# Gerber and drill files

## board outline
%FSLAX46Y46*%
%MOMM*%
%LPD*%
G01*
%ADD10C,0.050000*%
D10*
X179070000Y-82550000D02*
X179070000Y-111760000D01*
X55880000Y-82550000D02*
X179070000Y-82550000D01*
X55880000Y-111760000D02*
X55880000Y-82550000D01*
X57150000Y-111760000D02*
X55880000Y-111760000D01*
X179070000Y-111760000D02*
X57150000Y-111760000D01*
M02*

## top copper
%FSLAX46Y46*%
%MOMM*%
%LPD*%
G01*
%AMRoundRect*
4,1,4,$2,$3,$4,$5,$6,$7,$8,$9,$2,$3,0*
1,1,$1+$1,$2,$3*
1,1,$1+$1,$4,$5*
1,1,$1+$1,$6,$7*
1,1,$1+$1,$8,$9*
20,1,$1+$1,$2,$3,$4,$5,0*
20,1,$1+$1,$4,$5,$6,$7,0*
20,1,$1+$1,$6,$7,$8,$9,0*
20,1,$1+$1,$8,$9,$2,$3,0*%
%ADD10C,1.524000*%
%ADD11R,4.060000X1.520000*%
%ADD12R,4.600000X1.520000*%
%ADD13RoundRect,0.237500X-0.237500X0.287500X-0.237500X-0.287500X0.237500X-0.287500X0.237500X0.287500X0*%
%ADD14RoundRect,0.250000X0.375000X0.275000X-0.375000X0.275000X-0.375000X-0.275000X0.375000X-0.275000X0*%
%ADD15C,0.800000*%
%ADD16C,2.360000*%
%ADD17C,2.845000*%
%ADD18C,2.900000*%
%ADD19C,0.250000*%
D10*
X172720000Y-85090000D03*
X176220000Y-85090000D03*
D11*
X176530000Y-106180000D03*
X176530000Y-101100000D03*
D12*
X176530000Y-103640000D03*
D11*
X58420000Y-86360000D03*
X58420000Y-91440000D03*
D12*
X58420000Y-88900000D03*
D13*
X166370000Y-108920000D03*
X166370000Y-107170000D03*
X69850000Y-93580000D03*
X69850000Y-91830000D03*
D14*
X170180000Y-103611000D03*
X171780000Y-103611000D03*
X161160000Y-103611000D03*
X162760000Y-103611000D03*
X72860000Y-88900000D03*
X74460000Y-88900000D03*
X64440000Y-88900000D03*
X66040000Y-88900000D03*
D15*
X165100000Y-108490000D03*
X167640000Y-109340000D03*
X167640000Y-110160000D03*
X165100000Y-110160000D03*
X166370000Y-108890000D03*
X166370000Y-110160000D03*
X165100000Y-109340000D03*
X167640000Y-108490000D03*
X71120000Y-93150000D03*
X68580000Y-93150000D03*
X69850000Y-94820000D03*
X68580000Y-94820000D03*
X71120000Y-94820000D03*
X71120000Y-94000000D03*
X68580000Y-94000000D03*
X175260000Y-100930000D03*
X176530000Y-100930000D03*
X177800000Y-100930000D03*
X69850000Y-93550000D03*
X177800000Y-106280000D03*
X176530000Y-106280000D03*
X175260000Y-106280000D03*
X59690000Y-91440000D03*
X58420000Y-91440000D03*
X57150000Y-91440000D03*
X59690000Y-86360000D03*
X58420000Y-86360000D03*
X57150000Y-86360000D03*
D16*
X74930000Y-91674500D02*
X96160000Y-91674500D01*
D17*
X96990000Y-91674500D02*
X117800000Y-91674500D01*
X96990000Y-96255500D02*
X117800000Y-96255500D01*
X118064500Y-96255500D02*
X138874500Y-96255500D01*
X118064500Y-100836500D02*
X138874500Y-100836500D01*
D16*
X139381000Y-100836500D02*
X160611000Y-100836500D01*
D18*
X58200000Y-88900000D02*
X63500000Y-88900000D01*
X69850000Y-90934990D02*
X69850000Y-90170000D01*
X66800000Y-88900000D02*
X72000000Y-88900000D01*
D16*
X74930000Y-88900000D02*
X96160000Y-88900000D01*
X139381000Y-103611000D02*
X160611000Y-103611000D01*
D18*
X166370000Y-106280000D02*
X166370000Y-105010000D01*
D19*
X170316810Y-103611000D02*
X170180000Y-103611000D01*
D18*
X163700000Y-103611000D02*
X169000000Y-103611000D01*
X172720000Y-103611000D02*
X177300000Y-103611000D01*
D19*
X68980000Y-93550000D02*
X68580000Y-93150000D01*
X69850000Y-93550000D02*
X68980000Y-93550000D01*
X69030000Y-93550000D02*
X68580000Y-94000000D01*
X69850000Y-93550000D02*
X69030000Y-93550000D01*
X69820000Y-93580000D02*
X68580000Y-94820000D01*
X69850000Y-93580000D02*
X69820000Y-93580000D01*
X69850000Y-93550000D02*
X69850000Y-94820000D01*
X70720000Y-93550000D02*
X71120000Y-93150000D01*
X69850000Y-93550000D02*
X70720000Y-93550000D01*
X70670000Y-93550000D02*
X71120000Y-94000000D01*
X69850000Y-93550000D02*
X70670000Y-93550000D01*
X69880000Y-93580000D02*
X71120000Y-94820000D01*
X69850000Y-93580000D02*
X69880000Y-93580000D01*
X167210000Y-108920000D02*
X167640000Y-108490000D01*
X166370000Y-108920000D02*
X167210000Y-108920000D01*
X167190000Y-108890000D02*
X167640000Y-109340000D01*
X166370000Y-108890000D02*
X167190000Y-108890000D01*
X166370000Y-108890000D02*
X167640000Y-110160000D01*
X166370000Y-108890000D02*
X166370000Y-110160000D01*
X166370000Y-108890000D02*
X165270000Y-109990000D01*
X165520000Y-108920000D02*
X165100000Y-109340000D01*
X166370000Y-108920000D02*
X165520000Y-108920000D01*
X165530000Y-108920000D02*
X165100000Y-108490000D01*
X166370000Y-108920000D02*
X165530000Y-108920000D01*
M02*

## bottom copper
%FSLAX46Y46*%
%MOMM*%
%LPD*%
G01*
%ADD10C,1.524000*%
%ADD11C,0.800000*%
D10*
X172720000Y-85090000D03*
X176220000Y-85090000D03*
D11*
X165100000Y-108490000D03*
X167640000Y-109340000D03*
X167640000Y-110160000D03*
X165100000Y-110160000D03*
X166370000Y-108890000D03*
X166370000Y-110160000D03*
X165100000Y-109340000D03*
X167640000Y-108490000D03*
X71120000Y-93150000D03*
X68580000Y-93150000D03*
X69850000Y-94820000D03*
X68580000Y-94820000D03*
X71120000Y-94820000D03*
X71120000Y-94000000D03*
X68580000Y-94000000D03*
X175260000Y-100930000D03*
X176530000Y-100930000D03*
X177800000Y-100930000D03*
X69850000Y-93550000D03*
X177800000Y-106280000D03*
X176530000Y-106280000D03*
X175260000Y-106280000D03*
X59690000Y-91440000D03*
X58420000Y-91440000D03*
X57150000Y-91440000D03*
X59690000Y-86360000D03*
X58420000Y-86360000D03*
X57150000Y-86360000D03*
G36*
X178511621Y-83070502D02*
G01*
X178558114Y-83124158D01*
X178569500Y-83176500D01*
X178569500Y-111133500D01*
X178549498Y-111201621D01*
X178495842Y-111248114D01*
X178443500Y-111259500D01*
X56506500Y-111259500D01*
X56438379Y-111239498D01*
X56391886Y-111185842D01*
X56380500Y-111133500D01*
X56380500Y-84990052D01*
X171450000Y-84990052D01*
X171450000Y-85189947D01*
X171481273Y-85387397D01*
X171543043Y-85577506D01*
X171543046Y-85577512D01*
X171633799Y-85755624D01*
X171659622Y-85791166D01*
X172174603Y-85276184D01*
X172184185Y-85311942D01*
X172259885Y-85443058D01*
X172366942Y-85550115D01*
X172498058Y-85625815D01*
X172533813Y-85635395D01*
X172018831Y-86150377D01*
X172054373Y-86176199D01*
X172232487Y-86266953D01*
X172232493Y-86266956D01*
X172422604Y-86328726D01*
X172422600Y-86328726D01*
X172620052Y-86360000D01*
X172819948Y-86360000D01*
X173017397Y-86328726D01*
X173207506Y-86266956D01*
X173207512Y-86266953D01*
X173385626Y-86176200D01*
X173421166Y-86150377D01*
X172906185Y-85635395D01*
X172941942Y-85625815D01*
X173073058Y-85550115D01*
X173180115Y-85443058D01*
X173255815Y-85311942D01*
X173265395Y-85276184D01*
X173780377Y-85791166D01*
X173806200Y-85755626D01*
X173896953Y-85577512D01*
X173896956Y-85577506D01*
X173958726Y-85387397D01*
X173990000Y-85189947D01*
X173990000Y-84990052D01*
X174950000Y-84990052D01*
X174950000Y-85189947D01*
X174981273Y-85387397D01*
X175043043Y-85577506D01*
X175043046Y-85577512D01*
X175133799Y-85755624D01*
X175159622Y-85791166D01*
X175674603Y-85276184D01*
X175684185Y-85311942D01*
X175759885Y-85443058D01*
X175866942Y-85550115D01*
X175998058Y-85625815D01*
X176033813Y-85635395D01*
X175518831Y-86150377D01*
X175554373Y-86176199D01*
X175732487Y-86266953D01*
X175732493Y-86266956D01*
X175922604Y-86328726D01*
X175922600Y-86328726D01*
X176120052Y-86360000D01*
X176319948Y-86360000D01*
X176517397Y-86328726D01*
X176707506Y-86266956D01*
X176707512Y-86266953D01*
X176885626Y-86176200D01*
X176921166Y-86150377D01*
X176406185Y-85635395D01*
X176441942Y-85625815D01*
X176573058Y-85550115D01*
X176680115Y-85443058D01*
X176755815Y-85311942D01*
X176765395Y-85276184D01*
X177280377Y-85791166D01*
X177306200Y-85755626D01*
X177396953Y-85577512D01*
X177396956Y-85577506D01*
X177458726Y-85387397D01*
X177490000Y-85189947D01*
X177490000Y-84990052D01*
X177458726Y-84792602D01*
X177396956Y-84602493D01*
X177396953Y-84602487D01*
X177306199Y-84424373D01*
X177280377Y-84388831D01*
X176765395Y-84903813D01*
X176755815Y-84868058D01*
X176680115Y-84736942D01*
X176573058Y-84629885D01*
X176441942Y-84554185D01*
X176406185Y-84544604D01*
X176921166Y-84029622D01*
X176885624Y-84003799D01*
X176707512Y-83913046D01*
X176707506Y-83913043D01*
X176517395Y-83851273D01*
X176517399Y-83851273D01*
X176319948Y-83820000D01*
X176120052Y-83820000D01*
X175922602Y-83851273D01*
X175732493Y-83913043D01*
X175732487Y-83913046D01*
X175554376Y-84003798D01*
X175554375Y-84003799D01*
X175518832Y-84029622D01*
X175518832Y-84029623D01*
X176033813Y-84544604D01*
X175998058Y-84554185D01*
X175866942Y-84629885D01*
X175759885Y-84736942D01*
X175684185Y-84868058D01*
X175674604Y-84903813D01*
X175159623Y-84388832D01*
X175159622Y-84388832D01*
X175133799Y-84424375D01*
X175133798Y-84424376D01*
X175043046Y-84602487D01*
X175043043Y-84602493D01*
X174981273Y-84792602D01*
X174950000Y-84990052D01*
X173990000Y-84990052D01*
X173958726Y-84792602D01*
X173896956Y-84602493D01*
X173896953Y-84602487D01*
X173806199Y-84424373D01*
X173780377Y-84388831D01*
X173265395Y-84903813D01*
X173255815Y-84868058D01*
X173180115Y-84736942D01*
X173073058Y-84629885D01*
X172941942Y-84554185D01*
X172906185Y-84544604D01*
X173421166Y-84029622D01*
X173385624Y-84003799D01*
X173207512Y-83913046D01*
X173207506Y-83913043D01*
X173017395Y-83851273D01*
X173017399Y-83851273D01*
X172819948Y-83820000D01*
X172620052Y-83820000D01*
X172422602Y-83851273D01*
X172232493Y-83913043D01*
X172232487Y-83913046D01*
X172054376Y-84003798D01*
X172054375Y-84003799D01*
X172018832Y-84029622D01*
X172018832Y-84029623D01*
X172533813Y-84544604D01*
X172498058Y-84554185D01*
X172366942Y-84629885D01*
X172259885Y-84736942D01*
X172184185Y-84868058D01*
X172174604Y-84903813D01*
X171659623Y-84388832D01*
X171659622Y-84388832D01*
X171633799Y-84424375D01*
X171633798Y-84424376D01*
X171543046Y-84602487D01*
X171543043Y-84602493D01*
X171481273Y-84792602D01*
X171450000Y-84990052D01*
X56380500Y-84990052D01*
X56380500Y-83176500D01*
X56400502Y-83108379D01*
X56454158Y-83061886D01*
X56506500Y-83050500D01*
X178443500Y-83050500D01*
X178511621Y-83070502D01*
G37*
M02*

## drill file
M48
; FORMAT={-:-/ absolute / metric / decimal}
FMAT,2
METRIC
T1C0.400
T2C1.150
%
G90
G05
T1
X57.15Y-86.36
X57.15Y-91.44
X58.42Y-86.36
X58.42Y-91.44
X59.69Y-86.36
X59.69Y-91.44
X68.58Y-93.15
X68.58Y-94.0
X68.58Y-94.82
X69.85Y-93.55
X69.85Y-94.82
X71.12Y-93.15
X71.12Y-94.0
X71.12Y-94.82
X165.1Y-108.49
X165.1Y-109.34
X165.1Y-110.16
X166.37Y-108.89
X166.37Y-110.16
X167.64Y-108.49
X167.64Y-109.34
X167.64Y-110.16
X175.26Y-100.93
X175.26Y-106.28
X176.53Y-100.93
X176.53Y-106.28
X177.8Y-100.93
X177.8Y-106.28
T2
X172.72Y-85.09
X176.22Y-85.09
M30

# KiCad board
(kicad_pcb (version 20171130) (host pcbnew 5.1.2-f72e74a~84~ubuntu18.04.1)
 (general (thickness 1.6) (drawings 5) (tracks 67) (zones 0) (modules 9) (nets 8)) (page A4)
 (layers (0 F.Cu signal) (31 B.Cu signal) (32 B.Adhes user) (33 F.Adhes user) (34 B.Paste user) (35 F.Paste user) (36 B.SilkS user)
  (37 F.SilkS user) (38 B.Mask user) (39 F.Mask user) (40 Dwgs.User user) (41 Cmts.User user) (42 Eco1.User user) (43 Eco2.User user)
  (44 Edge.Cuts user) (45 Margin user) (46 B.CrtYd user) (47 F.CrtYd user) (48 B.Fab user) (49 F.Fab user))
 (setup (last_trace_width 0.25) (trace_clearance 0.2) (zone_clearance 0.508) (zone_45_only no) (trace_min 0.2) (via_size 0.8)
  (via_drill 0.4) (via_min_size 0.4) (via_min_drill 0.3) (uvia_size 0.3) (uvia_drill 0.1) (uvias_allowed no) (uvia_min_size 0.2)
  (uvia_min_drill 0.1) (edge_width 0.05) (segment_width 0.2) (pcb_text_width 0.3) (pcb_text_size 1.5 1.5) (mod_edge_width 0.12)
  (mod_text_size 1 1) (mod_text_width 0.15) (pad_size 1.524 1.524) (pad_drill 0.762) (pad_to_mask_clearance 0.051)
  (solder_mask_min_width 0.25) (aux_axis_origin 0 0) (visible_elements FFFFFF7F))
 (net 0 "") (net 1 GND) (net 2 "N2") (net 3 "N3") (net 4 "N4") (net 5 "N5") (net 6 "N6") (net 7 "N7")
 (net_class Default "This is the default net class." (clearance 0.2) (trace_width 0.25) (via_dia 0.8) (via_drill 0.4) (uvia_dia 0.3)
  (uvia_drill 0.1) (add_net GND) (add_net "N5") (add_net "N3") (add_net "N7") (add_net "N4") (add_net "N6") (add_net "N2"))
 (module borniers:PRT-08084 (layer F.Cu) (at 172.72 80.01 180)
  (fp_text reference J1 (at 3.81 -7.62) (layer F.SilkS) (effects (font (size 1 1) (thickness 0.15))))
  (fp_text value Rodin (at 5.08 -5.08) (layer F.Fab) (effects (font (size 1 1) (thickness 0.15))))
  (pad 2 thru_hole circle (at 0 -5.08 180) (size 1.524 1.524) (drill 1.15) (layers *.Cu *.Mask) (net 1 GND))
  (pad 1 thru_hole circle (at -3.5 -5.08 180) (size 1.524 1.524) (drill 1.15) (layers *.Cu *.Mask) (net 1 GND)))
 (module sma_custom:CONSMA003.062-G (layer F.Cu) (at 180.34 106.18)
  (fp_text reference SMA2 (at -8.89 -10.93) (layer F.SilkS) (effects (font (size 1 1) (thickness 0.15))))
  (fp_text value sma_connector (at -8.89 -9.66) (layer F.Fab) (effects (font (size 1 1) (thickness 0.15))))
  (pad 3 smd rect (at -3.81 0) (size 4.06 1.52) (layers F.Cu F.Paste F.Mask) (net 1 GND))
  (pad 2 smd rect (at -3.81 -5.08) (size 4.06 1.52) (layers F.Cu F.Paste F.Mask) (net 1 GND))
  (pad 1 smd rect (at -3.81 -2.54) (size 4.6 1.52) (layers F.Cu F.Paste F.Mask) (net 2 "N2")))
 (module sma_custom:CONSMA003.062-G (layer F.Cu) (at 54.61 86.36 180)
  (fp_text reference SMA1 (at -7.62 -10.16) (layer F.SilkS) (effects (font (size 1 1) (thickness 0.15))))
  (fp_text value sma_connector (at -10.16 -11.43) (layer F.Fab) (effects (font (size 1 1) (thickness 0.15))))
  (pad 3 smd rect (at -3.81 0 180) (size 4.06 1.52) (layers F.Cu F.Paste F.Mask) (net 1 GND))
  (pad 2 smd rect (at -3.81 -5.08 180) (size 4.06 1.52) (layers F.Cu F.Paste F.Mask) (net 1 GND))
  (pad 1 smd rect (at -3.81 -2.54 180) (size 4.6 1.52) (layers F.Cu F.Paste F.Mask) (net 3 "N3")))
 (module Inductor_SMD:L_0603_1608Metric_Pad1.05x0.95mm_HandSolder (layer F.Cu) (at 166.37 108.045 270)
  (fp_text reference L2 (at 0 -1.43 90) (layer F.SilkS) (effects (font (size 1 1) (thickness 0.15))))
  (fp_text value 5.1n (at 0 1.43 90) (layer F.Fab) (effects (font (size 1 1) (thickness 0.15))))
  (pad 2 smd roundrect (at 0.875 0 270) (size 1.05 0.95) (layers F.Cu F.Paste F.Mask) (roundrect_rratio 0.25) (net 1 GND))
  (pad 1 smd roundrect (at -0.875 0 270) (size 1.05 0.95) (layers F.Cu F.Paste F.Mask) (roundrect_rratio 0.25) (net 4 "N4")))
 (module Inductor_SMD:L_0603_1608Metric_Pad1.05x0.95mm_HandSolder (layer F.Cu) (at 69.85 92.705 270)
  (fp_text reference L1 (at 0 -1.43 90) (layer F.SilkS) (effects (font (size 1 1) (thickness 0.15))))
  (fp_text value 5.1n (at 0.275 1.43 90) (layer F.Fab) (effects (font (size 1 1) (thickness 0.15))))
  (pad 2 smd roundrect (at 0.875 0 270) (size 1.05 0.95) (layers F.Cu F.Paste F.Mask) (roundrect_rratio 0.25) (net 1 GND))
  (pad 1 smd roundrect (at -0.875 0 270) (size 1.05 0.95) (layers F.Cu F.Paste F.Mask) (roundrect_rratio 0.25) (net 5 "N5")))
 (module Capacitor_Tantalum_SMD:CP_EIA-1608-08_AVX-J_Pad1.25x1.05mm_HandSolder (layer F.Cu) (at 170.98 103.611 180)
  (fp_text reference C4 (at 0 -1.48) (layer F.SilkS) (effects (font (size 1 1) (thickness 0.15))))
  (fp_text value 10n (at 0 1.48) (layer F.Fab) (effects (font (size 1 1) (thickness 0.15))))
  (pad 2 smd roundrect (at 0.8 0 180) (size 1.25 1.05) (layers F.Cu F.Paste F.Mask) (roundrect_rratio 0.238095) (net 4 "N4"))
  (pad 1 smd roundrect (at -0.8 0 180) (size 1.25 1.05) (layers F.Cu F.Paste F.Mask) (roundrect_rratio 0.238095) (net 2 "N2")))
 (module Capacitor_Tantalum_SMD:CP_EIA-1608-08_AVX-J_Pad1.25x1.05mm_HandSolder (layer F.Cu) (at 161.96 103.611 180)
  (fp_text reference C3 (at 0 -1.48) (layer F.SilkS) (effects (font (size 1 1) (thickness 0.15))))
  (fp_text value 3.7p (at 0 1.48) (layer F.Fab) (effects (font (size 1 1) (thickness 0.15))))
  (pad 2 smd roundrect (at 0.8 0 180) (size 1.25 1.05) (layers F.Cu F.Paste F.Mask) (roundrect_rratio 0.238095) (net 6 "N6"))
  (pad 1 smd roundrect (at -0.8 0 180) (size 1.25 1.05) (layers F.Cu F.Paste F.Mask) (roundrect_rratio 0.238095) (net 4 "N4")))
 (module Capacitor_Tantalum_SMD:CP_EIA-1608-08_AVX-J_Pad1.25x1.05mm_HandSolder (layer F.Cu) (at 73.66 88.9 180)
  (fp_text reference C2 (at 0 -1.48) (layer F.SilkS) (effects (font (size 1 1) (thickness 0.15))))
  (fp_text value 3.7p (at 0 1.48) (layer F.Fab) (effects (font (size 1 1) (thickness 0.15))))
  (pad 2 smd roundrect (at 0.8 0 180) (size 1.25 1.05) (layers F.Cu F.Paste F.Mask) (roundrect_rratio 0.238095) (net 5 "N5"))
  (pad 1 smd roundrect (at -0.8 0 180) (size 1.25 1.05) (layers F.Cu F.Paste F.Mask) (roundrect_rratio 0.238095) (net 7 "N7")))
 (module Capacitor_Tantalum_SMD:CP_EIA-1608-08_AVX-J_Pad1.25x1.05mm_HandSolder (layer F.Cu) (at 65.24 88.9 180)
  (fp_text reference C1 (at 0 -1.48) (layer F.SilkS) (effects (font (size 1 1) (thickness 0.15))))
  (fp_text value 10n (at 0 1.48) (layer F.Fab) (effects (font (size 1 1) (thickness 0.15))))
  (pad 2 smd roundrect (at 0.8 0 180) (size 1.25 1.05) (layers F.Cu F.Paste F.Mask) (roundrect_rratio 0.238095) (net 3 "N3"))
  (pad 1 smd roundrect (at -0.8 0 180) (size 1.25 1.05) (layers F.Cu F.Paste F.Mask) (roundrect_rratio 0.238095) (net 5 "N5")))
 (gr_line (start 179.07 82.55) (end 179.07 111.76) (layer Edge.Cuts) (width 0.05))
 (gr_line (start 55.88 82.55) (end 179.07 82.55) (layer Edge.Cuts) (width 0.05))
 (gr_line (start 55.88 111.76) (end 55.88 82.55) (layer Edge.Cuts) (width 0.05))
 (gr_line (start 57.15 111.76) (end 55.88 111.76) (layer Edge.Cuts) (width 0.05))
 (gr_line (start 179.07 111.76) (end 57.15 111.76) (layer Edge.Cuts) (width 0.05))
 (segment (start 74.93 91.6745) (end 96.16 91.6745) (width 2.36) (layer F.Cu) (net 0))
 (segment (start 96.99 91.6745) (end 117.8 91.6745) (width 2.845) (layer F.Cu) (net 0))
 (segment (start 96.99 96.2555) (end 117.8 96.2555) (width 2.845) (layer F.Cu) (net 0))
 (segment (start 118.0645 96.2555) (end 138.8745 96.2555) (width 2.845) (layer F.Cu) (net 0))
 (segment (start 118.0645 100.8365) (end 138.8745 100.8365) (width 2.845) (layer F.Cu) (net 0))
 (segment (start 139.381 100.8365) (end 160.611 100.8365) (width 2.36) (layer F.Cu) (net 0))
 (segment (start 58.2 88.9) (end 63.5 88.9) (width 2.9) (layer F.Cu) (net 3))
 (segment (start 69.85 90.93499) (end 69.85 90.17) (width 2.9) (layer F.Cu) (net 5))
 (segment (start 66.8 88.9) (end 72 88.9) (width 2.9) (layer F.Cu) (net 5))
 (segment (start 74.93 88.9) (end 96.16 88.9) (width 2.36) (layer F.Cu) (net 7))
 (segment (start 139.381 103.611) (end 160.611 103.611) (width 2.36) (layer F.Cu) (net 6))
 (segment (start 166.37 106.28) (end 166.37 105.01) (width 2.9) (layer F.Cu) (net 4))
 (segment (start 170.31681 103.611) (end 170.18 103.611) (width 0.25) (layer F.Cu) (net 4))
 (segment (start 163.7 103.611) (end 169 103.611) (width 2.9) (layer F.Cu) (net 4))
 (segment (start 172.72 103.611) (end 177.3 103.611) (width 2.9) (layer F.Cu) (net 2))
 (via (at 165.1 108.49) (size 0.8) (drill 0.4) (layers F.Cu B.Cu) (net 1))
 (via (at 167.64 109.34) (size 0.8) (drill 0.4) (layers F.Cu B.Cu) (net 1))
 (via (at 167.64 110.16) (size 0.8) (drill 0.4) (layers F.Cu B.Cu) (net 1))
 (via (at 165.1 110.16) (size 0.8) (drill 0.4) (layers F.Cu B.Cu) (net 1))
 (via (at 166.37 108.89) (size 0.8) (drill 0.4) (layers F.Cu B.Cu) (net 1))
 (via (at 166.37 110.16) (size 0.8) (drill 0.4) (layers F.Cu B.Cu) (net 1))
 (via (at 165.1 109.34) (size 0.8) (drill 0.4) (layers F.Cu B.Cu) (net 1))
 (via (at 167.64 108.49) (size 0.8) (drill 0.4) (layers F.Cu B.Cu) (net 1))
 (via (at 71.12 93.15) (size 0.8) (drill 0.4) (layers F.Cu B.Cu) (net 1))
 (via (at 68.58 93.15) (size 0.8) (drill 0.4) (layers F.Cu B.Cu) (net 1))
 (via (at 69.85 94.82) (size 0.8) (drill 0.4) (layers F.Cu B.Cu) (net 1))
 (via (at 68.58 94.82) (size 0.8) (drill 0.4) (layers F.Cu B.Cu) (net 1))
 (via (at 71.12 94.82) (size 0.8) (drill 0.4) (layers F.Cu B.Cu) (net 1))
 (via (at 71.12 94) (size 0.8) (drill 0.4) (layers F.Cu B.Cu) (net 1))
 (via (at 68.58 94) (size 0.8) (drill 0.4) (layers F.Cu B.Cu) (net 1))
 (via (at 175.26 100.93) (size 0.8) (drill 0.4) (layers F.Cu B.Cu) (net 1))
 (via (at 176.53 100.93) (size 0.8) (drill 0.4) (layers F.Cu B.Cu) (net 1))
 (via (at 177.8 100.93) (size 0.8) (drill 0.4) (layers F.Cu B.Cu) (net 1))
 (via (at 69.85 93.55) (size 0.8) (drill 0.4) (layers F.Cu B.Cu) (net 1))
 (via (at 177.8 106.28) (size 0.8) (drill 0.4) (layers F.Cu B.Cu) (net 1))
 (via (at 176.53 106.28) (size 0.8) (drill 0.4) (layers F.Cu B.Cu) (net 1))
 (via (at 175.26 106.28) (size 0.8) (drill 0.4) (layers F.Cu B.Cu) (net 1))
 (via (at 59.69 91.44) (size 0.8) (drill 0.4) (layers F.Cu B.Cu) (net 1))
 (via (at 58.42 91.44) (size 0.8) (drill 0.4) (layers F.Cu B.Cu) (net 1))
 (via (at 57.15 91.44) (size 0.8) (drill 0.4) (layers F.Cu B.Cu) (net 1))
 (via (at 59.69 86.36) (size 0.8) (drill 0.4) (layers F.Cu B.Cu) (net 1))
 (via (at 58.42 86.36) (size 0.8) (drill 0.4) (layers F.Cu B.Cu) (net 1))
 (via (at 57.15 86.36) (size 0.8) (drill 0.4) (layers F.Cu B.Cu) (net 1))
 (segment (start 68.98 93.55) (end 68.58 93.15) (width 0.25) (layer F.Cu) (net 1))
 (segment (start 69.85 93.55) (end 68.98 93.55) (width 0.25) (layer F.Cu) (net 1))
 (segment (start 69.03 93.55) (end 68.58 94) (width 0.25) (layer F.Cu) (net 1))
 (segment (start 69.85 93.55) (end 69.03 93.55) (width 0.25) (layer F.Cu) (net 1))
 (segment (start 69.82 93.58) (end 68.58 94.82) (width 0.25) (layer F.Cu) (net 1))
 (segment (start 69.85 93.58) (end 69.82 93.58) (width 0.25) (layer F.Cu) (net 1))
 (segment (start 69.85 93.55) (end 69.85 94.82) (width 0.25) (layer F.Cu) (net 1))
 (segment (start 70.72 93.55) (end 71.12 93.15) (width 0.25) (layer F.Cu) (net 1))
 (segment (start 69.85 93.55) (end 70.72 93.55) (width 0.25) (layer F.Cu) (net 1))
 (segment (start 70.67 93.55) (end 71.12 94) (width 0.25) (layer F.Cu) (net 1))
 (segment (start 69.85 93.55) (end 70.67 93.55) (width 0.25) (layer F.Cu) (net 1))
 (segment (start 69.88 93.58) (end 71.12 94.82) (width 0.25) (layer F.Cu) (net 1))
 (segment (start 69.85 93.58) (end 69.88 93.58) (width 0.25) (layer F.Cu) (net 1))
 (segment (start 167.21 108.92) (end 167.64 108.49) (width 0.25) (layer F.Cu) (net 1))
 (segment (start 166.37 108.92) (end 167.21 108.92) (width 0.25) (layer F.Cu) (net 1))
 (segment (start 167.19 108.89) (end 167.64 109.34) (width 0.25) (layer F.Cu) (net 1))
 (segment (start 166.37 108.89) (end 167.19 108.89) (width 0.25) (layer F.Cu) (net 1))
 (segment (start 166.37 108.89) (end 167.64 110.16) (width 0.25) (layer F.Cu) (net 1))
 (segment (start 166.37 108.89) (end 166.37 110.16) (width 0.25) (layer F.Cu) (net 1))
 (segment (start 166.37 108.89) (end 165.27 109.99) (width 0.25) (layer F.Cu) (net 1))
 (segment (start 165.52 108.92) (end 165.1 109.34) (width 0.25) (layer F.Cu) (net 1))
 (segment (start 166.37 108.92) (end 165.52 108.92) (width 0.25) (layer F.Cu) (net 1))
 (segment (start 165.53 108.92) (end 165.1 108.49) (width 0.25) (layer F.Cu) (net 1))
 (segment (start 166.37 108.92) (end 165.53 108.92) (width 0.25) (layer F.Cu) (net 1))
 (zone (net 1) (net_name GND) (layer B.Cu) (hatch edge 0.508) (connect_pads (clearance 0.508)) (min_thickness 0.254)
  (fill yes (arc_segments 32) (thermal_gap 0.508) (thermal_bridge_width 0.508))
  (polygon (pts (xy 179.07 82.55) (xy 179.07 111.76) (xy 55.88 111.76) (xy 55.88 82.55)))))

